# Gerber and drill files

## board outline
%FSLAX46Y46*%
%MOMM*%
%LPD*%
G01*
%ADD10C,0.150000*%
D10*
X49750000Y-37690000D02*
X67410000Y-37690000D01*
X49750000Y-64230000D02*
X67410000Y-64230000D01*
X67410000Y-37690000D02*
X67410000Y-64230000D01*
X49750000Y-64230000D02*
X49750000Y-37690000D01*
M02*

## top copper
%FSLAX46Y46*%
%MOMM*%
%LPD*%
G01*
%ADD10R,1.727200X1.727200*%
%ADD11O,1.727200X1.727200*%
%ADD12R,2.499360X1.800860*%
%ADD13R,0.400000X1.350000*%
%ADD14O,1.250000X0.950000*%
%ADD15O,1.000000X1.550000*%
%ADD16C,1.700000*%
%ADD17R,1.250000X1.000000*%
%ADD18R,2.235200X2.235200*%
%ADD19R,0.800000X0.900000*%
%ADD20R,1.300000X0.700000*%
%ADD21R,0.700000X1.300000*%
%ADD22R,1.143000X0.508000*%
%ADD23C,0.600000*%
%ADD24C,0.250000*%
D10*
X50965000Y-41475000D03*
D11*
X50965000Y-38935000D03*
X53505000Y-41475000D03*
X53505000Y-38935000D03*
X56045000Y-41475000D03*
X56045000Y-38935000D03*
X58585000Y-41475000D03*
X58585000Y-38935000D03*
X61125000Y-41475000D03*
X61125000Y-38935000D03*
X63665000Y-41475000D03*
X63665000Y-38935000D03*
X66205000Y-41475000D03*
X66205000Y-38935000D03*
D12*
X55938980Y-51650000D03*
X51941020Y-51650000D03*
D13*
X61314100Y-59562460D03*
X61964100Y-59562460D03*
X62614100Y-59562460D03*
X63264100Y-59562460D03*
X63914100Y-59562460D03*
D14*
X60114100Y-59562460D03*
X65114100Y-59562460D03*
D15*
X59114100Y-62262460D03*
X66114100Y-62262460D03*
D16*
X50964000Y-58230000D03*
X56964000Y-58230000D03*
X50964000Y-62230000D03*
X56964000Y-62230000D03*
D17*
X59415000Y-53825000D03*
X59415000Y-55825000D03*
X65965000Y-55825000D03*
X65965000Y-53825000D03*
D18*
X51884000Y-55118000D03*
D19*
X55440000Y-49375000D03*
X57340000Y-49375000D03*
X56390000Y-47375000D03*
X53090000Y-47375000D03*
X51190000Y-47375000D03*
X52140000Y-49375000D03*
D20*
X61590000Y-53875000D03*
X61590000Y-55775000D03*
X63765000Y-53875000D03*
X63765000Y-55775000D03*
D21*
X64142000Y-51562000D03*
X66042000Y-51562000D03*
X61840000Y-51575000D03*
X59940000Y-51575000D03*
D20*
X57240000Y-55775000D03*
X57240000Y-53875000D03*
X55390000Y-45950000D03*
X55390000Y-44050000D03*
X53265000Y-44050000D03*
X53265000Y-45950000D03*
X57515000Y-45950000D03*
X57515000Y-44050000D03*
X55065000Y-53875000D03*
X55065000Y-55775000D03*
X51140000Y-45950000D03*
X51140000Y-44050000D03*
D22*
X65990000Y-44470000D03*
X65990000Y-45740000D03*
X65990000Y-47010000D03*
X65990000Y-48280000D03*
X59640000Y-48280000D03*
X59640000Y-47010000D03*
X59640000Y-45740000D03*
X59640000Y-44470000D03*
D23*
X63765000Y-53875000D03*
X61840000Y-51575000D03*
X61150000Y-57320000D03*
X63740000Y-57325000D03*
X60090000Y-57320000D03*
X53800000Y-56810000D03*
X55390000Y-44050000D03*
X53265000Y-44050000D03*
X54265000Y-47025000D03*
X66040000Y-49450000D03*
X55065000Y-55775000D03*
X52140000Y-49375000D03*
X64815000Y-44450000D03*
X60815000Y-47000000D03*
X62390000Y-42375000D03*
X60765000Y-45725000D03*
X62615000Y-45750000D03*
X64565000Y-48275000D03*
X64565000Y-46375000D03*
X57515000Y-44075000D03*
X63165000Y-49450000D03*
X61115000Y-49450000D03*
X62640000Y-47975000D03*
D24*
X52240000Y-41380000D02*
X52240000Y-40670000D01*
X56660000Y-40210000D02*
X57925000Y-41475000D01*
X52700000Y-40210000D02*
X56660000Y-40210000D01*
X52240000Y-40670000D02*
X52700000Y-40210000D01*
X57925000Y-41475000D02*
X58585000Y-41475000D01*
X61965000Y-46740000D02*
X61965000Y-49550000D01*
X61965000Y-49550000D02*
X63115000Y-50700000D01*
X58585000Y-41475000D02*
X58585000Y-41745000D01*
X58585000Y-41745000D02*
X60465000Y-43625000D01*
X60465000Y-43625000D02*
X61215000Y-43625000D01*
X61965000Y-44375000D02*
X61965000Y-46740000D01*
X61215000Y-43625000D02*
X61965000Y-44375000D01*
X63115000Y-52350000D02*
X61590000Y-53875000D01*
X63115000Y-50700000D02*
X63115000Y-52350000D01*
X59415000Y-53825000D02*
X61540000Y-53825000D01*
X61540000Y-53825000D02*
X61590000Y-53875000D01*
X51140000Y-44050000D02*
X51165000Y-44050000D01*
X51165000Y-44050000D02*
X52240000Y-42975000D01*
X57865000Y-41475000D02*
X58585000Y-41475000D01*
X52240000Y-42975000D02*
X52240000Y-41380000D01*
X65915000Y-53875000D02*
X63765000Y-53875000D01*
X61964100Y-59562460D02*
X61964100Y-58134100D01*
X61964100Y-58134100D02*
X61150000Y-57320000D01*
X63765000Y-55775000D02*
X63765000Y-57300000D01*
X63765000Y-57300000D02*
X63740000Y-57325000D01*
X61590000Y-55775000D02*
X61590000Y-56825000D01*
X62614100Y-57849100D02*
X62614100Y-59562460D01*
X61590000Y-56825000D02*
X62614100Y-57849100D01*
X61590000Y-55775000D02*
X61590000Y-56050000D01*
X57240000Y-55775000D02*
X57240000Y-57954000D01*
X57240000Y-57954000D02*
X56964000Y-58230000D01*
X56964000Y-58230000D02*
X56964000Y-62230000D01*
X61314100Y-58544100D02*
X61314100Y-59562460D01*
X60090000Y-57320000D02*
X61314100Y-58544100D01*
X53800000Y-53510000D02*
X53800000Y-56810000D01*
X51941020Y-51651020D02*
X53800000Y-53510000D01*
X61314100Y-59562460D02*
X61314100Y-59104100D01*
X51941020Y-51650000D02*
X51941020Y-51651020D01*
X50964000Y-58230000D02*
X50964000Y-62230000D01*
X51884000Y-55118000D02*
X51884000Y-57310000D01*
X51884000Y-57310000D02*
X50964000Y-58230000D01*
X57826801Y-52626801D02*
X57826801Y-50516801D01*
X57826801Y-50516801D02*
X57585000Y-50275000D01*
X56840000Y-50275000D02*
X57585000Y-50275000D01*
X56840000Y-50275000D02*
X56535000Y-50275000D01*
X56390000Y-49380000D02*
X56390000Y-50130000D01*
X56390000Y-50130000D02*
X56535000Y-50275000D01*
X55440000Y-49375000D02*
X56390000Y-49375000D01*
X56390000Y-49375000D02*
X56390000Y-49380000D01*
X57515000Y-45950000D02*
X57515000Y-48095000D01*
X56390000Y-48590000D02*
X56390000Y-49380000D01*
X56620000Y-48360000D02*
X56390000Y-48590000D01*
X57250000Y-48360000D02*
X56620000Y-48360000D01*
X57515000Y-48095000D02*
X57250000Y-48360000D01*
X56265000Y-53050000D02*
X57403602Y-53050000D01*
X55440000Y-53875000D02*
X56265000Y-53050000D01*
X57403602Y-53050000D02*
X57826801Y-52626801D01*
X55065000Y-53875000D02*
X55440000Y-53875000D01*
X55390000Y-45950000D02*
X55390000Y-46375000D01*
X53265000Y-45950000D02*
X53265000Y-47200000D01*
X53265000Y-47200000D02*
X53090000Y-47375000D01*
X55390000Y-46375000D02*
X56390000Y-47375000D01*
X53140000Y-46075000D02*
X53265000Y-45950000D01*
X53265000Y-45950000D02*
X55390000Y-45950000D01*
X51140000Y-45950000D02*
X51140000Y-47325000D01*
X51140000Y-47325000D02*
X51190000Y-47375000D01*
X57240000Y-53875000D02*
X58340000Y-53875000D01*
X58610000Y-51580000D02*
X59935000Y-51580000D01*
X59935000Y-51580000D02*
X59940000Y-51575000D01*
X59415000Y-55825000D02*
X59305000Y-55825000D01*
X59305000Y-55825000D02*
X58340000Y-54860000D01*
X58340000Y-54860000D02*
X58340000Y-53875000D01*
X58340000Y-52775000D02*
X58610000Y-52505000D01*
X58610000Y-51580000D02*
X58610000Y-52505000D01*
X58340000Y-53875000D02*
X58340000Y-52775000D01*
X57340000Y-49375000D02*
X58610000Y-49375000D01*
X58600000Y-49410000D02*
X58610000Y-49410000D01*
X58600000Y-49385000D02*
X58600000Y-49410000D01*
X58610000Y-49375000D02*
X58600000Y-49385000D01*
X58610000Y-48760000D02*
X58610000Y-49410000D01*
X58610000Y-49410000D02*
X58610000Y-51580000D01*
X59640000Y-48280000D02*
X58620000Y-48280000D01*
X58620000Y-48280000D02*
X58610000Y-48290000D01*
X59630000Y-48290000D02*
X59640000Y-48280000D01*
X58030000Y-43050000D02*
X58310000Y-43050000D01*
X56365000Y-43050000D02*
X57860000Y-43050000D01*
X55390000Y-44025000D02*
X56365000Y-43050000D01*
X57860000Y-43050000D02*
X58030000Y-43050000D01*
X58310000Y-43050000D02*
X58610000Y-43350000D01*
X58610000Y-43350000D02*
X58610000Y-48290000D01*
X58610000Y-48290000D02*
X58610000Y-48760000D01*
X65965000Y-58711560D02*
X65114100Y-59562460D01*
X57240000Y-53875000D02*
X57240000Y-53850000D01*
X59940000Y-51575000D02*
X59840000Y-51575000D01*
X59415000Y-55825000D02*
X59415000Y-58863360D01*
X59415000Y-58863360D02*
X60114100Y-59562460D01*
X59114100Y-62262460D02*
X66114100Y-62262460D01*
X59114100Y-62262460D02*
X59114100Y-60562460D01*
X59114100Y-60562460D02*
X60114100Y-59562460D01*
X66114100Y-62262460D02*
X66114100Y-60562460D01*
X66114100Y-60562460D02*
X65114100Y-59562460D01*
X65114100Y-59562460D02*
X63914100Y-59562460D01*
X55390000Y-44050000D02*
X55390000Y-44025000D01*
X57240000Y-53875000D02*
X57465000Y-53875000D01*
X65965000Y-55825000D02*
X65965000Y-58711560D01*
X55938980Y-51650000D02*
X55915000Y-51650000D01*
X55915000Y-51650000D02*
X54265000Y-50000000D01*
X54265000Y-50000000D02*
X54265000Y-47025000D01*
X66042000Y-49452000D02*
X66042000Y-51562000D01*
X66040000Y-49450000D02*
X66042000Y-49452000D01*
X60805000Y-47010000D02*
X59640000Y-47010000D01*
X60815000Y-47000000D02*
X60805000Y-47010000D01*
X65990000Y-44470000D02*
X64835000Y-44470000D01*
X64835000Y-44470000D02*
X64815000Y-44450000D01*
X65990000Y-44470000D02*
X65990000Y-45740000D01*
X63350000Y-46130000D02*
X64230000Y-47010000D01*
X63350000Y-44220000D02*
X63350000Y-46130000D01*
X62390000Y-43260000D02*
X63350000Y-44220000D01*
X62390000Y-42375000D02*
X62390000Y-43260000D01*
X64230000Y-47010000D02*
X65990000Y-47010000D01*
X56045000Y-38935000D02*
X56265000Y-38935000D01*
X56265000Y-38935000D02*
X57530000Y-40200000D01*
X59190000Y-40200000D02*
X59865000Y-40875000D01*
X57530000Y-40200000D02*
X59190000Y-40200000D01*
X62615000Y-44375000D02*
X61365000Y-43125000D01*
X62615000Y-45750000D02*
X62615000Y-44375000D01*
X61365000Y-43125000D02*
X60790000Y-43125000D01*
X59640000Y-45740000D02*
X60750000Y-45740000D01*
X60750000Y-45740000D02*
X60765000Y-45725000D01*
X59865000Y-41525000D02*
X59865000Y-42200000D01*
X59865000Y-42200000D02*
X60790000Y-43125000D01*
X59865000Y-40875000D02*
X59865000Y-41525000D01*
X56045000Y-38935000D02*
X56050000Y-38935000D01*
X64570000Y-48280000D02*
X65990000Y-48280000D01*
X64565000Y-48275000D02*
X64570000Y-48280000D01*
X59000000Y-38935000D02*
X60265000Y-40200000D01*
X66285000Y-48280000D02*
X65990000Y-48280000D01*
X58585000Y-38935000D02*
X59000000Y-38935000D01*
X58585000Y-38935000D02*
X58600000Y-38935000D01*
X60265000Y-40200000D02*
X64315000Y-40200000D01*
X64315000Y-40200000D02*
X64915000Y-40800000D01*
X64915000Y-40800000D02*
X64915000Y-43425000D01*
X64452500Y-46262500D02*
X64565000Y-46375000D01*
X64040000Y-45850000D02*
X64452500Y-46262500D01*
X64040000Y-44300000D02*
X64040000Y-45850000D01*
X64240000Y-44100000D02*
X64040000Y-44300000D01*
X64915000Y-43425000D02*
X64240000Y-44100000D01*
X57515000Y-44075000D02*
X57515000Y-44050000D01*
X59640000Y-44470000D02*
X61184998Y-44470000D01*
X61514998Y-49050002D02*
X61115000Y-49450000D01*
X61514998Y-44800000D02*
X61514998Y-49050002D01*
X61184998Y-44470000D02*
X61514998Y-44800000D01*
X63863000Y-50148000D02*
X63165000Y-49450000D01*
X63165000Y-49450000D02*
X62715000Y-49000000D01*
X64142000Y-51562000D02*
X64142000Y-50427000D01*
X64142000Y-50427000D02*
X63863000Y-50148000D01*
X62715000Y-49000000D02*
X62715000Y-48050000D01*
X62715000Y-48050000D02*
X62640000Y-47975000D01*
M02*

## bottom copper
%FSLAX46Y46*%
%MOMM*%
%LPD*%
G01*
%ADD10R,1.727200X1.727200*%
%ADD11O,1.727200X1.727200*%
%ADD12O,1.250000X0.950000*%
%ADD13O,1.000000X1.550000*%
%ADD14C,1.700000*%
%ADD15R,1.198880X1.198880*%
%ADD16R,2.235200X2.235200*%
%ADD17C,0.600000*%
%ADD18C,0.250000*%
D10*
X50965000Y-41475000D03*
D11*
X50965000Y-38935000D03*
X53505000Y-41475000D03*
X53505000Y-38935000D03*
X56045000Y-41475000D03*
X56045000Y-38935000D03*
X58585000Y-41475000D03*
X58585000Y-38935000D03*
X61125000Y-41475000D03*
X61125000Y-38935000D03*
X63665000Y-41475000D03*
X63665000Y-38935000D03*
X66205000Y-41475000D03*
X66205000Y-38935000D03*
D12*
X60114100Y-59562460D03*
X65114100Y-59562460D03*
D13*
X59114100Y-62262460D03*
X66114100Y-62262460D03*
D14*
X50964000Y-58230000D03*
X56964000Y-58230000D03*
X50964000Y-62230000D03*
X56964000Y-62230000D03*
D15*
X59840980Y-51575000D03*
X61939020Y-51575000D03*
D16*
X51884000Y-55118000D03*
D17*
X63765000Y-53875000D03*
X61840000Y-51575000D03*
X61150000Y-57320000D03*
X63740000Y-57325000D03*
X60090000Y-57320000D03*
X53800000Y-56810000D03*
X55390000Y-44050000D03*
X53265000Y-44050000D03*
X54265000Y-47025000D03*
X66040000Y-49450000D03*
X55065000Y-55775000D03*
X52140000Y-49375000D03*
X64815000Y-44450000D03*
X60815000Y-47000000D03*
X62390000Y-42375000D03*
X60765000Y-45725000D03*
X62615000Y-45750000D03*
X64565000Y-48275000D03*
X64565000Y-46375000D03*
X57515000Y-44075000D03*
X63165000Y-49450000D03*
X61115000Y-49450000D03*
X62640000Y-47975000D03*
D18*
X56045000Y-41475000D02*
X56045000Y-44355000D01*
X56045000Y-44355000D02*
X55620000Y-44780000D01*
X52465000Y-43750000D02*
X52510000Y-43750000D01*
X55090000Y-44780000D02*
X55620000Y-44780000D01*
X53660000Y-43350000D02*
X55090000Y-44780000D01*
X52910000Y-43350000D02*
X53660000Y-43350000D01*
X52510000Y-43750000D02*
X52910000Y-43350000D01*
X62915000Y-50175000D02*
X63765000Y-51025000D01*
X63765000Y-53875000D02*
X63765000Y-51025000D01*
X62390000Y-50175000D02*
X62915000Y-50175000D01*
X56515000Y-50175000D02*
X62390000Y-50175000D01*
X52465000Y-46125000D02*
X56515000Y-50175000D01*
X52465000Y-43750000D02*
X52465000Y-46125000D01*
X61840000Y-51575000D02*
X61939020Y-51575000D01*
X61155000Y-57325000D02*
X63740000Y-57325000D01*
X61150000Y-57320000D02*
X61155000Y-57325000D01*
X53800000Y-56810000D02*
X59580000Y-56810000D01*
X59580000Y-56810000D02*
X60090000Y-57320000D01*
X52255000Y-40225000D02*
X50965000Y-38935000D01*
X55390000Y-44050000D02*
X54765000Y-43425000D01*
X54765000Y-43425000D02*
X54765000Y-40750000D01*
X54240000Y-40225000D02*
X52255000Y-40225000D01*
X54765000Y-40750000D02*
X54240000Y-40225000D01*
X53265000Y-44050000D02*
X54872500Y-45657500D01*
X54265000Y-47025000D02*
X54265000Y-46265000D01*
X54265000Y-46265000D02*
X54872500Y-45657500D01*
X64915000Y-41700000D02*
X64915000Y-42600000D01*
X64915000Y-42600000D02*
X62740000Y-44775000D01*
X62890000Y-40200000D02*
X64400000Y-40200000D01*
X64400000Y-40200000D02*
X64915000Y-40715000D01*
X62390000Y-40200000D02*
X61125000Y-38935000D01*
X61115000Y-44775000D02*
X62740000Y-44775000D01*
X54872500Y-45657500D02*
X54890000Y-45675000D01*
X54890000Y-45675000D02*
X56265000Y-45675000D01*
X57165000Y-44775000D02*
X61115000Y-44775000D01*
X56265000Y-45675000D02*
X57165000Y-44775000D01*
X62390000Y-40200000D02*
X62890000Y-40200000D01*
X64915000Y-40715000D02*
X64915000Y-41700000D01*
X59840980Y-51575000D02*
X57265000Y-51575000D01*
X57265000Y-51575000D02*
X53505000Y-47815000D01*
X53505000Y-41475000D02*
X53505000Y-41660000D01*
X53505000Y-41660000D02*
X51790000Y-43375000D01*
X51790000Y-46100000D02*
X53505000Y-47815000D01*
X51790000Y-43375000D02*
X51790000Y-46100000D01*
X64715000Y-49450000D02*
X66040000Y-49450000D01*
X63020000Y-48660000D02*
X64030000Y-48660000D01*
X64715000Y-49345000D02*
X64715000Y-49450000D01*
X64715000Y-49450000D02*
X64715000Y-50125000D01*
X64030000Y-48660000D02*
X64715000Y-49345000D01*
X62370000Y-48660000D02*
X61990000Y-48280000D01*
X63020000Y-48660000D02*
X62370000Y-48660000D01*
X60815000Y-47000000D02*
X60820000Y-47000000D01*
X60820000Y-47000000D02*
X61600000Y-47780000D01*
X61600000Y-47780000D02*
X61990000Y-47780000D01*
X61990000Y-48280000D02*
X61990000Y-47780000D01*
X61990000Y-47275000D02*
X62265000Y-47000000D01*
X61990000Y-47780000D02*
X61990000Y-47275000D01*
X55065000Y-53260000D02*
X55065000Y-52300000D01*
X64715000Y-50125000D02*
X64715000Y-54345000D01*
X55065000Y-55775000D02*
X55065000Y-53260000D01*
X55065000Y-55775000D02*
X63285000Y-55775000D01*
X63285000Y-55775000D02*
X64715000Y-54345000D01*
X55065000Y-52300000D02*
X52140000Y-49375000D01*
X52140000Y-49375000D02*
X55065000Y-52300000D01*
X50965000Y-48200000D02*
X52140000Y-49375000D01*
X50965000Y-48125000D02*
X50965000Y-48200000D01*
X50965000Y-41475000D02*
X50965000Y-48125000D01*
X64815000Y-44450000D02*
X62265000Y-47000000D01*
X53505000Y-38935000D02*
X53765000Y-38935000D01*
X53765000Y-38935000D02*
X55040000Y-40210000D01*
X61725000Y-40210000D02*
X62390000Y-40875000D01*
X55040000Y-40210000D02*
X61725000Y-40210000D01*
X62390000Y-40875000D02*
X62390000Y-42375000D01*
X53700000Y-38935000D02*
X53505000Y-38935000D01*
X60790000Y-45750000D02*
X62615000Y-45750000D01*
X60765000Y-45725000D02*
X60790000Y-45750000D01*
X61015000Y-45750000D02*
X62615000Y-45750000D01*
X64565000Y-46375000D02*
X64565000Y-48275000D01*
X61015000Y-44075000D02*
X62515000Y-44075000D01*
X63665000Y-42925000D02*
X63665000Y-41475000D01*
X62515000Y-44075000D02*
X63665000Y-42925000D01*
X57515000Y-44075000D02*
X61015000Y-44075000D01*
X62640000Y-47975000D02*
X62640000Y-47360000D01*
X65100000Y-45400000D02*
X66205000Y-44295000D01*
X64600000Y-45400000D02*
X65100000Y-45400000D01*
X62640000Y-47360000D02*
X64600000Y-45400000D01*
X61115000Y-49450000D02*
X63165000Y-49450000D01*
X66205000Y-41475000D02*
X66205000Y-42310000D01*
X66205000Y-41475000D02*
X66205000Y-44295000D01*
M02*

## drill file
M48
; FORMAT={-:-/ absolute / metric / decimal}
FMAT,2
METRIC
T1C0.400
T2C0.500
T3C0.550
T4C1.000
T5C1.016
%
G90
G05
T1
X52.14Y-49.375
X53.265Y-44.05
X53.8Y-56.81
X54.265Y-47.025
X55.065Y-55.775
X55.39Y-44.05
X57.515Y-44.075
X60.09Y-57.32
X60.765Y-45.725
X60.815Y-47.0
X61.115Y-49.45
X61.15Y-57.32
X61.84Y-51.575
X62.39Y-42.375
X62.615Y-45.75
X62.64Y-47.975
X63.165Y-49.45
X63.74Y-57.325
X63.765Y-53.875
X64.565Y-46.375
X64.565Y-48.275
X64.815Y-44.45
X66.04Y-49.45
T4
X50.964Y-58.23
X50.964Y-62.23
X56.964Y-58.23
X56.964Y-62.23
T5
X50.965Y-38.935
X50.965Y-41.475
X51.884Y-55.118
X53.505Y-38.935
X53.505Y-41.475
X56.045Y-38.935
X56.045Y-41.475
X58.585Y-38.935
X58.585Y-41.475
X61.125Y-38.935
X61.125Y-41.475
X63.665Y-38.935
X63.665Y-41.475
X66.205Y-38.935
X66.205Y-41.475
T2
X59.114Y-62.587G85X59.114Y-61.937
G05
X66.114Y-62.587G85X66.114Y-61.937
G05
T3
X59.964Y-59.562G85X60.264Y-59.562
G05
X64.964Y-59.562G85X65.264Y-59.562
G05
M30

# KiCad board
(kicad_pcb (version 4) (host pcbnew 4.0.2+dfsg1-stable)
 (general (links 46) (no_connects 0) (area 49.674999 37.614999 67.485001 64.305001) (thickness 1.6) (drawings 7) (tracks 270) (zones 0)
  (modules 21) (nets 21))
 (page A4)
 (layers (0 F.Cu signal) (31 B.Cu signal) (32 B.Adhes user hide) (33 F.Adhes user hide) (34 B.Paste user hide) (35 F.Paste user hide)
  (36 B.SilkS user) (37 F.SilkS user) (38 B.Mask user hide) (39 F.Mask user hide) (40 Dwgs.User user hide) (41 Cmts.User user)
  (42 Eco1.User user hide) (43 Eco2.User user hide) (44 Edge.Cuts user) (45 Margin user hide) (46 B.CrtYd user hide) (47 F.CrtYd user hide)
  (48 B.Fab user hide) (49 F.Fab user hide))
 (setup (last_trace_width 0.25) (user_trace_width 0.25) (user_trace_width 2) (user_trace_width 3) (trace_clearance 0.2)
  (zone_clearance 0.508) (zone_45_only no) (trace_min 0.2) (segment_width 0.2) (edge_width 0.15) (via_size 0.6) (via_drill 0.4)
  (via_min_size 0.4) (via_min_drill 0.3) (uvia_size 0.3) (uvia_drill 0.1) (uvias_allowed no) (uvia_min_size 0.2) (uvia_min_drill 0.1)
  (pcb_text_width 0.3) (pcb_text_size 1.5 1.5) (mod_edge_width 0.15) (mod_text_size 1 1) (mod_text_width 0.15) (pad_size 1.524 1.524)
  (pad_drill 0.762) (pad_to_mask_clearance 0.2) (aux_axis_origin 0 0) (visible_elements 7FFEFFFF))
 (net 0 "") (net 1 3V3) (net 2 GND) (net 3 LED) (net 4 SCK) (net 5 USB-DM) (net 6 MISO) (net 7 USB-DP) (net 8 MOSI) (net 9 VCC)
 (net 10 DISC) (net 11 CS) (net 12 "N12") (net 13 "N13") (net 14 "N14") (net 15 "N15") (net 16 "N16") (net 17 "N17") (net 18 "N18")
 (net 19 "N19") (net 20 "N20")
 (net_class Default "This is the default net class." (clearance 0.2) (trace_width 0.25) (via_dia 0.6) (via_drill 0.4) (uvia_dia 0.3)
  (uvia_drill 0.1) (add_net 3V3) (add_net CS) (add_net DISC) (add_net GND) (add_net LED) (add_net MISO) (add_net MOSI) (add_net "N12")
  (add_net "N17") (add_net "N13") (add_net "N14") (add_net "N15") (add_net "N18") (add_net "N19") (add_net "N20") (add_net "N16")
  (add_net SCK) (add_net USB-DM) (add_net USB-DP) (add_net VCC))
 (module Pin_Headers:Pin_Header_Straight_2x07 (layer F.Cu) (at 50.965 41.475 90)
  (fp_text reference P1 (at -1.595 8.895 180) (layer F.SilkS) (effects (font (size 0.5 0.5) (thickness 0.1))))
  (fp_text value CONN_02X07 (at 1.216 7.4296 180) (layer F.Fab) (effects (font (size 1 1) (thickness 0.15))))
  (pad 1 thru_hole rect (at 0 0 90) (size 1.7272 1.7272) (drill 1.016) (layers *.Cu *.Mask) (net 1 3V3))
  (pad 2 thru_hole oval (at 2.54 0 90) (size 1.7272 1.7272) (drill 1.016) (layers *.Cu *.Mask) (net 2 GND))
  (pad 3 thru_hole oval (at 0 2.54 90) (size 1.7272 1.7272) (drill 1.016) (layers *.Cu *.Mask) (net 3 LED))
  (pad 4 thru_hole oval (at 2.54 2.54 90) (size 1.7272 1.7272) (drill 1.016) (layers *.Cu *.Mask) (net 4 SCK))
  (pad 5 thru_hole oval (at 0 5.08 90) (size 1.7272 1.7272) (drill 1.016) (layers *.Cu *.Mask) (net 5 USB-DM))
  (pad 6 thru_hole oval (at 2.54 5.08 90) (size 1.7272 1.7272) (drill 1.016) (layers *.Cu *.Mask) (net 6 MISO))
  (pad 7 thru_hole oval (at 0 7.62 90) (size 1.7272 1.7272) (drill 1.016) (layers *.Cu *.Mask) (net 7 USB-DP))
  (pad 8 thru_hole oval (at 2.54 7.62 90) (size 1.7272 1.7272) (drill 1.016) (layers *.Cu *.Mask) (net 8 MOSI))
  (pad 9 thru_hole oval (at 0 10.16 90) (size 1.7272 1.7272) (drill 1.016) (layers *.Cu *.Mask))
  (pad 10 thru_hole oval (at 2.54 10.16 90) (size 1.7272 1.7272) (drill 1.016) (layers *.Cu *.Mask) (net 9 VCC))
  (pad 11 thru_hole oval (at 0 12.7 90) (size 1.7272 1.7272) (drill 1.016) (layers *.Cu *.Mask) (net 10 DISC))
  (pad 12 thru_hole oval (at 2.54 12.7 90) (size 1.7272 1.7272) (drill 1.016) (layers *.Cu *.Mask))
  (pad 13 thru_hole oval (at 0 15.24 90) (size 1.7272 1.7272) (drill 1.016) (layers *.Cu *.Mask) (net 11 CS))
  (pad 14 thru_hole oval (at 2.54 15.24 90) (size 1.7272 1.7272) (drill 1.016) (layers *.Cu *.Mask)))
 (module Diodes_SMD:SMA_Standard (layer F.Cu) (at 53.94 51.65 180)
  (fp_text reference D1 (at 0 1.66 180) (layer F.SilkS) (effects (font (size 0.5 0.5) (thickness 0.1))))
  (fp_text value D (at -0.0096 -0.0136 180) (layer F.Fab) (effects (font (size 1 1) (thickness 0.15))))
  (pad 1 smd rect (at -1.99898 0 180) (size 2.49936 1.80086) (layers F.Cu F.Paste F.Mask) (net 9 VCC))
  (pad 2 smd rect (at 1.99898 0 180) (size 2.49936 1.80086) (layers F.Cu F.Paste F.Mask) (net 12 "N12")))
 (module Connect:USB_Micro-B (layer F.Cu) (at 62.615 61.125)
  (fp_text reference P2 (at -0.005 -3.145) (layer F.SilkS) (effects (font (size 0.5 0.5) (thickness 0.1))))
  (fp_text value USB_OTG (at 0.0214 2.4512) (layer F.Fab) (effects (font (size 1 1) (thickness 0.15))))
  (pad 1 smd rect (at -1.3009 -1.56254 90) (size 1.35 0.4) (layers F.Cu F.Paste F.Mask) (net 12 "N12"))
  (pad 2 smd rect (at -0.6509 -1.56254 90) (size 1.35 0.4) (layers F.Cu F.Paste F.Mask) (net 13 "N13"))
  (pad 3 smd rect (at -0.0009 -1.56254 90) (size 1.35 0.4) (layers F.Cu F.Paste F.Mask) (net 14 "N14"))
  (pad 4 smd rect (at 0.6491 -1.56254 90) (size 1.35 0.4) (layers F.Cu F.Paste F.Mask))
  (pad 5 smd rect (at 1.2991 -1.56254 90) (size 1.35 0.4) (layers F.Cu F.Paste F.Mask) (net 2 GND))
  (pad 6 thru_hole oval (at -2.5009 -1.56254 90) (size 0.95 1.25) (drill oval 0.55 0.85) (layers *.Cu *.Mask) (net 2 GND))
  (pad 6 thru_hole oval (at 2.4991 -1.56254 90) (size 0.95 1.25) (drill oval 0.55 0.85) (layers *.Cu *.Mask) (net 2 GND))
  (pad 6 thru_hole oval (at -3.5009 1.13746 90) (size 1.55 1) (drill oval 1.15 0.5) (layers *.Cu *.Mask) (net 2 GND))
  (pad 6 thru_hole oval (at 3.4991 1.13746 90) (size 1.55 1) (drill oval 1.15 0.5) (layers *.Cu *.Mask) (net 2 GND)))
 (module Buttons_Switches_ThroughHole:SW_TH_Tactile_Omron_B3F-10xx (layer F.Cu) (at 56.964 62.23 180)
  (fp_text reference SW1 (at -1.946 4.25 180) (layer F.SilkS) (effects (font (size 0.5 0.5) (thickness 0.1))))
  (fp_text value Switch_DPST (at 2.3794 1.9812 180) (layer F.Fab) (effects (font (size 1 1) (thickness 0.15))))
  (pad 4 thru_hole circle (at 6 4 180) (size 1.7 1.7) (drill 1) (layers *.Cu *.Mask) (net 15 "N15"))
  (pad 3 thru_hole circle (at 0 4 180) (size 1.7 1.7) (drill 1) (layers *.Cu *.Mask) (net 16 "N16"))
  (pad 2 thru_hole circle (at 6 0 180) (size 1.7 1.7) (drill 1) (layers *.Cu *.Mask) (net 15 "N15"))
  (pad 1 thru_hole circle (at 0 0 180) (size 1.7 1.7) (drill 1) (layers *.Cu *.Mask) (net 16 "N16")))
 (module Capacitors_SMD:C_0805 (layer F.Cu) (at 59.415 54.825 270)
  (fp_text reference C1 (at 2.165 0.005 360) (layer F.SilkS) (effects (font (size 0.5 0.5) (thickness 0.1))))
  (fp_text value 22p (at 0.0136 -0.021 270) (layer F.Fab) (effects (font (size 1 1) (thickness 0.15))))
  (pad 1 smd rect (at -1 0 270) (size 1 1.25) (layers F.Cu F.Paste F.Mask) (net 7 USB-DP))
  (pad 2 smd rect (at 1 0 270) (size 1 1.25) (layers F.Cu F.Paste F.Mask) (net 2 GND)))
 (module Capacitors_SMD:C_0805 (layer F.Cu) (at 65.965 54.825 90)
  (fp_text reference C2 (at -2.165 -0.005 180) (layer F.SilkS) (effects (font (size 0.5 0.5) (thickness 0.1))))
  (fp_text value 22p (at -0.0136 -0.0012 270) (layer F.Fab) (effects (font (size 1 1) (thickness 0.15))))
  (pad 1 smd rect (at -1 0 90) (size 1 1.25) (layers F.Cu F.Paste F.Mask) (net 2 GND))
  (pad 2 smd rect (at 1 0 90) (size 1 1.25) (layers F.Cu F.Paste F.Mask) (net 5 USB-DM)))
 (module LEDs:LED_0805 (layer B.Cu) (at 60.89 51.575 180)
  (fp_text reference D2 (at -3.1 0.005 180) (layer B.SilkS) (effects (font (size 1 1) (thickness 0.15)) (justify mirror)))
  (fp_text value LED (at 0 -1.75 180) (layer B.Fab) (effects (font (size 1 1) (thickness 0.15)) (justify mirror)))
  (pad 2 smd rect (at 1.04902 0) (size 1.19888 1.19888) (layers B.Cu B.Paste B.Mask) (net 3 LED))
  (pad 1 smd rect (at -1.04902 0) (size 1.19888 1.19888) (layers B.Cu B.Paste B.Mask) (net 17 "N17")))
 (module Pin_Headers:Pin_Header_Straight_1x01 (layer F.Cu) (at 51.884 55.118)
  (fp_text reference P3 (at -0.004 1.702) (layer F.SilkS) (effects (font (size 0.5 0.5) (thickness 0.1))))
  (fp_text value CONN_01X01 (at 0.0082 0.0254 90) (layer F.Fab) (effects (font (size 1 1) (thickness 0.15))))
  (pad 1 thru_hole rect (at 0 0) (size 2.2352 2.2352) (drill 1.016) (layers *.Cu *.Mask) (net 15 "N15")))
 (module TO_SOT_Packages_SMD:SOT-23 (layer F.Cu) (at 56.39 48.375 90)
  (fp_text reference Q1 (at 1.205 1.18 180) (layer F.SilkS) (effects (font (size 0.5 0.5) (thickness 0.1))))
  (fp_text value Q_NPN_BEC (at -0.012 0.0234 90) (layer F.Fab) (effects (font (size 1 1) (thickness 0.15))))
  (pad 1 smd rect (at -1 -0.95 90) (size 0.9 0.8) (layers F.Cu F.Paste F.Mask) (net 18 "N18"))
  (pad 2 smd rect (at -1 0.95 90) (size 0.9 0.8) (layers F.Cu F.Paste F.Mask) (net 2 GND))
  (pad 3 smd rect (at 1 0 90) (size 0.9 0.8) (layers F.Cu F.Paste F.Mask) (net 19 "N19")))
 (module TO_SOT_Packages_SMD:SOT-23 (layer F.Cu) (at 52.14 48.375 270)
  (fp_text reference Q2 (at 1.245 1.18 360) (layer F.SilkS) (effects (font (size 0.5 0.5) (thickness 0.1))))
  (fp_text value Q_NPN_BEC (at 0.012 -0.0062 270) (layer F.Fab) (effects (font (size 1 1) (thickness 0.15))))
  (pad 1 smd rect (at -1 -0.95 270) (size 0.9 0.8) (layers F.Cu F.Paste F.Mask) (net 19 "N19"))
  (pad 2 smd rect (at -1 0.95 270) (size 0.9 0.8) (layers F.Cu F.Paste F.Mask) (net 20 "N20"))
  (pad 3 smd rect (at 1 0 270) (size 0.9 0.8) (layers F.Cu F.Paste F.Mask) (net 1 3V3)))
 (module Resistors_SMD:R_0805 (layer F.Cu) (at 61.59 54.825 270)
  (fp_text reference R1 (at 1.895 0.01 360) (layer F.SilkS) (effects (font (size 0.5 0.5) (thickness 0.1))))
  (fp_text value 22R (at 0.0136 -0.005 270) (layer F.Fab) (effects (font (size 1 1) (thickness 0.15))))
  (pad 1 smd rect (at -0.95 0 270) (size 0.7 1.3) (layers F.Cu F.Paste F.Mask) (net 7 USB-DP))
  (pad 2 smd rect (at 0.95 0 270) (size 0.7 1.3) (layers F.Cu F.Paste F.Mask) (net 14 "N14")))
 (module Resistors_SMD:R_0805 (layer F.Cu) (at 63.765 54.825 270)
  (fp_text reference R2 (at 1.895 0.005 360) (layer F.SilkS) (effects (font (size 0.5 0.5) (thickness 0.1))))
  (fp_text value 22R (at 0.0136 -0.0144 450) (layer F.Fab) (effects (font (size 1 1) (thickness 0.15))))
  (pad 1 smd rect (at -0.95 0 270) (size 0.7 1.3) (layers F.Cu F.Paste F.Mask) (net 5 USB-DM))
  (pad 2 smd rect (at 0.95 0 270) (size 0.7 1.3) (layers F.Cu F.Paste F.Mask) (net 13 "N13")))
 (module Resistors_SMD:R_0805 (layer F.Cu) (at 65.092 51.562)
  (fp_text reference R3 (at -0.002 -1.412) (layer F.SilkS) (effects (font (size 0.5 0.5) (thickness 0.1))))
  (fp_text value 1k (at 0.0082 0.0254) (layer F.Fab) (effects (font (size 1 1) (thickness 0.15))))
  (pad 1 smd rect (at -0.95 0) (size 0.7 1.3) (layers F.Cu F.Paste F.Mask) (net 11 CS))
  (pad 2 smd rect (at 0.95 0) (size 0.7 1.3) (layers F.Cu F.Paste F.Mask) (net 1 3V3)))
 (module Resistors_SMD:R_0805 (layer F.Cu) (at 60.89 51.575 180)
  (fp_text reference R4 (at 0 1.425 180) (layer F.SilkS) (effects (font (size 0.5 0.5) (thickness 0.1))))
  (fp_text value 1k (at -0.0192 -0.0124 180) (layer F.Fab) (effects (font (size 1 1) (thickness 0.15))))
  (pad 1 smd rect (at -0.95 0 180) (size 0.7 1.3) (layers F.Cu F.Paste F.Mask) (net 17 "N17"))
  (pad 2 smd rect (at 0.95 0 180) (size 0.7 1.3) (layers F.Cu F.Paste F.Mask) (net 2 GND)))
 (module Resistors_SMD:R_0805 (layer F.Cu) (at 57.24 54.825 90)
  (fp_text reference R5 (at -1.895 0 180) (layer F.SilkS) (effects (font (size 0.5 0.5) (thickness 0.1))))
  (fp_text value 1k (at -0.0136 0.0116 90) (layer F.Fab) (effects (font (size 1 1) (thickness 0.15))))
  (pad 1 smd rect (at -0.95 0 90) (size 0.7 1.3) (layers F.Cu F.Paste F.Mask) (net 16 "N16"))
  (pad 2 smd rect (at 0.95 0 90) (size 0.7 1.3) (layers F.Cu F.Paste F.Mask) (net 2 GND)))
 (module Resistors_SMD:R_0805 (layer F.Cu) (at 55.39 45 90)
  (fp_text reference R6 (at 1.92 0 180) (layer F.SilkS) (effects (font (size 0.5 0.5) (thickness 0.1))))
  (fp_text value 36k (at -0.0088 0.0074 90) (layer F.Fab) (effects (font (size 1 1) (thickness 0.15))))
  (pad 1 smd rect (at -0.95 0 90) (size 0.7 1.3) (layers F.Cu F.Paste F.Mask) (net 19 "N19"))
  (pad 2 smd rect (at 0.95 0 90) (size 0.7 1.3) (layers F.Cu F.Paste F.Mask) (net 2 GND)))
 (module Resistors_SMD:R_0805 (layer F.Cu) (at 53.265 45 270)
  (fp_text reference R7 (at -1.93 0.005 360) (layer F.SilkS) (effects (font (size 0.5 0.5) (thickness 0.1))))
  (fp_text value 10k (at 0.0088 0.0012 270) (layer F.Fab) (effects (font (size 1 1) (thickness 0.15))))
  (pad 1 smd rect (at -0.95 0 270) (size 0.7 1.3) (layers F.Cu F.Paste F.Mask) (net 9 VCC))
  (pad 2 smd rect (at 0.95 0 270) (size 0.7 1.3) (layers F.Cu F.Paste F.Mask) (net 19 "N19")))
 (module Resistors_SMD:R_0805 (layer F.Cu) (at 57.515 45 90)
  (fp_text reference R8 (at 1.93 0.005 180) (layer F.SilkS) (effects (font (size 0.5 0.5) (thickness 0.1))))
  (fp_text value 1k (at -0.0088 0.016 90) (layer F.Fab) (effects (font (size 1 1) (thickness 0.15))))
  (pad 1 smd rect (at -0.95 0 90) (size 0.7 1.3) (layers F.Cu F.Paste F.Mask) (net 18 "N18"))
  (pad 2 smd rect (at 0.95 0 90) (size 0.7 1.3) (layers F.Cu F.Paste F.Mask) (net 10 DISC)))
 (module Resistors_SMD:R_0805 (layer F.Cu) (at 55.065 54.825 270)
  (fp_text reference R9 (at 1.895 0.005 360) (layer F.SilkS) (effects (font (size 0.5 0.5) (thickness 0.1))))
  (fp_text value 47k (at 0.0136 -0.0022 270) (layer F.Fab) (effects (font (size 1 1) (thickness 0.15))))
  (pad 1 smd rect (at -0.95 0 270) (size 0.7 1.3) (layers F.Cu F.Paste F.Mask) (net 18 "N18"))
  (pad 2 smd rect (at 0.95 0 270) (size 0.7 1.3) (layers F.Cu F.Paste F.Mask) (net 1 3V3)))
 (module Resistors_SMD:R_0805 (layer F.Cu) (at 51.14 45 90)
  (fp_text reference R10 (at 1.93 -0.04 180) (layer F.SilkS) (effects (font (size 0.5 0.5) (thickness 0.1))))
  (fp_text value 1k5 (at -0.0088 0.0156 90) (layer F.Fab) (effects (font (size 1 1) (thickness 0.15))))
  (pad 1 smd rect (at -0.95 0 90) (size 0.7 1.3) (layers F.Cu F.Paste F.Mask) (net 20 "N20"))
  (pad 2 smd rect (at 0.95 0 90) (size 0.7 1.3) (layers F.Cu F.Paste F.Mask) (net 7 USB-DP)))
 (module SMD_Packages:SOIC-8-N (layer F.Cu) (at 62.815 46.375 270)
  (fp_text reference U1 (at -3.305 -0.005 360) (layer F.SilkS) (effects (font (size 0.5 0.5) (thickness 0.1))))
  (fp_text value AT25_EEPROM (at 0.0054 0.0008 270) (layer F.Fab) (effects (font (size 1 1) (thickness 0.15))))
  (pad 8 smd rect (at -1.905 -3.175 270) (size 0.508 1.143) (layers F.Cu F.Paste F.Mask) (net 1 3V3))
  (pad 7 smd rect (at -0.635 -3.175 270) (size 0.508 1.143) (layers F.Cu F.Paste F.Mask) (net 1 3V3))
  (pad 6 smd rect (at 0.635 -3.175 270) (size 0.508 1.143) (layers F.Cu F.Paste F.Mask) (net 4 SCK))
  (pad 5 smd rect (at 1.905 -3.175 270) (size 0.508 1.143) (layers F.Cu F.Paste F.Mask) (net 8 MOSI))
  (pad 4 smd rect (at 1.905 3.175 270) (size 0.508 1.143) (layers F.Cu F.Paste F.Mask) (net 2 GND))
  (pad 3 smd rect (at 0.635 3.175 270) (size 0.508 1.143) (layers F.Cu F.Paste F.Mask) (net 1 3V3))
  (pad 2 smd rect (at -0.635 3.175 270) (size 0.508 1.143) (layers F.Cu F.Paste F.Mask) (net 6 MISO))
  (pad 1 smd rect (at -1.905 3.175 270) (size 0.508 1.143) (layers F.Cu F.Paste F.Mask) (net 11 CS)))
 (gr_line (start 49.75 37.69) (end 67.41 37.69) (angle 90) (layer Edge.Cuts) (width 0.15))
 (gr_line (start 49.75 64.23) (end 67.41 64.23) (angle 90) (layer Edge.Cuts) (width 0.15))
 (gr_line (start 67.41 37.69) (end 67.41 64.23) (angle 90) (layer Edge.Cuts) (width 0.15))
 (gr_line (start 49.75 64.23) (end 49.75 37.69) (angle 90) (layer Edge.Cuts) (width 0.15))
 (segment (start 52.24 41.38) (end 52.24 40.67) (width 0.25) (layer F.Cu) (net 7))
 (segment (start 56.66 40.21) (end 57.925 41.475) (width 0.25) (layer F.Cu) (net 7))
 (segment (start 52.7 40.21) (end 56.66 40.21) (width 0.25) (layer F.Cu) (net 7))
 (segment (start 52.24 40.67) (end 52.7 40.21) (width 0.25) (layer F.Cu) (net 7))
 (segment (start 57.925 41.475) (end 58.585 41.475) (width 0.25) (layer F.Cu) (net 7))
 (segment (start 61.965 46.74) (end 61.965 49.55) (width 0.25) (layer F.Cu) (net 7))
 (segment (start 61.965 49.55) (end 63.115 50.7) (width 0.25) (layer F.Cu) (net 7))
 (segment (start 58.585 41.475) (end 58.585 41.745) (width 0.25) (layer F.Cu) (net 7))
 (segment (start 58.585 41.745) (end 60.465 43.625) (width 0.25) (layer F.Cu) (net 7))
 (segment (start 60.465 43.625) (end 61.215 43.625) (width 0.25) (layer F.Cu) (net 7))
 (segment (start 61.965 44.375) (end 61.965 46.74) (width 0.25) (layer F.Cu) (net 7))
 (segment (start 61.215 43.625) (end 61.965 44.375) (width 0.25) (layer F.Cu) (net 7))
 (segment (start 63.115 52.35) (end 61.59 53.875) (width 0.25) (layer F.Cu) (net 7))
 (segment (start 63.115 50.7) (end 63.115 52.35) (width 0.25) (layer F.Cu) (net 7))
 (segment (start 59.415 53.825) (end 61.54 53.825) (width 0.25) (layer F.Cu) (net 7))
 (segment (start 61.54 53.825) (end 61.59 53.875) (width 0.25) (layer F.Cu) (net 7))
 (segment (start 51.14 44.05) (end 51.165 44.05) (width 0.25) (layer F.Cu) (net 7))
 (segment (start 51.165 44.05) (end 52.24 42.975) (width 0.25) (layer F.Cu) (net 7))
 (segment (start 57.865 41.475) (end 58.585 41.475) (width 0.25) (layer F.Cu) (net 7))
 (segment (start 52.24 42.975) (end 52.24 41.38) (width 0.25) (layer F.Cu) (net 7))
 (segment (start 56.045 41.475) (end 56.045 44.355) (width 0.25) (layer B.Cu) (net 5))
 (segment (start 56.045 44.355) (end 55.62 44.78) (width 0.25) (layer B.Cu) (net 5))
 (segment (start 52.465 43.75) (end 52.51 43.75) (width 0.25) (layer B.Cu) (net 5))
 (segment (start 55.09 44.78) (end 55.62 44.78) (width 0.25) (layer B.Cu) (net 5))
 (segment (start 53.66 43.35) (end 55.09 44.78) (width 0.25) (layer B.Cu) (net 5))
 (segment (start 52.91 43.35) (end 53.66 43.35) (width 0.25) (layer B.Cu) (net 5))
 (segment (start 52.51 43.75) (end 52.91 43.35) (width 0.25) (layer B.Cu) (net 5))
 (segment (start 62.915 50.175) (end 63.765 51.025) (width 0.25) (layer B.Cu) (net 5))
 (segment (start 63.765 53.875) (end 63.765 51.025) (width 0.25) (layer B.Cu) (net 5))
 (via (at 63.765 53.875) (size 0.6) (drill 0.4) (layers F.Cu B.Cu) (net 5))
 (segment (start 65.915 53.875) (end 63.765 53.875) (width 0.25) (layer F.Cu) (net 5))
 (segment (start 62.39 50.175) (end 62.915 50.175) (width 0.25) (layer B.Cu) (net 5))
 (segment (start 56.515 50.175) (end 62.39 50.175) (width 0.25) (layer B.Cu) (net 5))
 (segment (start 52.465 46.125) (end 56.515 50.175) (width 0.25) (layer B.Cu) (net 5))
 (segment (start 52.465 43.75) (end 52.465 46.125) (width 0.25) (layer B.Cu) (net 5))
 (via (at 61.84 51.575) (size 0.6) (drill 0.4) (layers F.Cu B.Cu) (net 17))
 (segment (start 61.84 51.575) (end 61.93902 51.575) (width 0.25) (layer B.Cu) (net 17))
 (segment (start 61.9641 59.56246) (end 61.9641 58.1341) (width 0.25) (layer F.Cu) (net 13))
 (segment (start 61.155 57.325) (end 63.74 57.325) (width 0.25) (layer B.Cu) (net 13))
 (segment (start 61.15 57.32) (end 61.155 57.325) (width 0.25) (layer B.Cu) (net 13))
 (via (at 61.15 57.32) (size 0.6) (drill 0.4) (layers F.Cu B.Cu) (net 13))
 (segment (start 61.9641 58.1341) (end 61.15 57.32) (width 0.25) (layer F.Cu) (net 13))
 (segment (start 63.765 55.775) (end 63.765 57.3) (width 0.25) (layer F.Cu) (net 13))
 (via (at 63.74 57.325) (size 0.6) (drill 0.4) (layers F.Cu B.Cu) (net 13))
 (segment (start 63.765 57.3) (end 63.74 57.325) (width 0.25) (layer F.Cu) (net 13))
 (segment (start 61.59 55.775) (end 61.59 56.825) (width 0.25) (layer F.Cu) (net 14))
 (segment (start 62.6141 57.8491) (end 62.6141 59.56246) (width 0.25) (layer F.Cu) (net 14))
 (segment (start 61.59 56.825) (end 62.6141 57.8491) (width 0.25) (layer F.Cu) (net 14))
 (segment (start 61.59 55.775) (end 61.59 56.05) (width 0.25) (layer F.Cu) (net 14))
 (segment (start 57.24 55.775) (end 57.24 57.954) (width 0.25) (layer F.Cu) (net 16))
 (segment (start 57.24 57.954) (end 56.964 58.23) (width 0.25) (layer F.Cu) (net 16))
 (segment (start 56.964 58.23) (end 56.964 62.23) (width 0.25) (layer F.Cu) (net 16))
 (segment (start 53.8 56.81) (end 59.58 56.81) (width 0.25) (layer B.Cu) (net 12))
 (segment (start 61.3141 58.5441) (end 61.3141 59.56246) (width 0.25) (layer F.Cu) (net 12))
 (segment (start 60.09 57.32) (end 61.3141 58.5441) (width 0.25) (layer F.Cu) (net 12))
 (via (at 60.09 57.32) (size 0.6) (drill 0.4) (layers F.Cu B.Cu) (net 12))
 (segment (start 59.58 56.81) (end 60.09 57.32) (width 0.25) (layer B.Cu) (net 12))
 (via (at 53.8 56.81) (size 0.6) (drill 0.4) (layers F.Cu B.Cu) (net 12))
 (segment (start 53.8 53.51) (end 53.8 56.81) (width 0.25) (layer F.Cu) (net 12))
 (segment (start 51.94102 51.65102) (end 53.8 53.51) (width 0.25) (layer F.Cu) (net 12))
 (segment (start 61.3141 59.56246) (end 61.3141 59.1041) (width 0.25) (layer F.Cu) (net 12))
 (segment (start 51.94102 51.65) (end 51.94102 51.65102) (width 0.25) (layer F.Cu) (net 12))
 (segment (start 50.964 58.23) (end 50.964 62.23) (width 0.25) (layer F.Cu) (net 15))
 (segment (start 51.884 55.118) (end 51.884 57.31) (width 0.25) (layer F.Cu) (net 15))
 (segment (start 51.884 57.31) (end 50.964 58.23) (width 0.25) (layer F.Cu) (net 15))
 (segment (start 57.826801 52.626801) (end 57.826801 50.516801) (width 0.25) (layer F.Cu) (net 18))
 (segment (start 57.826801 50.516801) (end 57.585 50.275) (width 0.25) (layer F.Cu) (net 18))
 (segment (start 56.84 50.275) (end 57.585 50.275) (width 0.25) (layer F.Cu) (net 18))
 (segment (start 56.84 50.275) (end 56.535 50.275) (width 0.25) (layer F.Cu) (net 18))
 (segment (start 56.39 49.38) (end 56.39 50.13) (width 0.25) (layer F.Cu) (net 18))
 (segment (start 56.39 50.13) (end 56.535 50.275) (width 0.25) (layer F.Cu) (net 18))
 (segment (start 55.44 49.375) (end 56.39 49.375) (width 0.25) (layer F.Cu) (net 18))
 (segment (start 56.39 49.375) (end 56.39 49.38) (width 0.25) (layer F.Cu) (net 18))
 (segment (start 57.515 45.95) (end 57.515 48.095) (width 0.25) (layer F.Cu) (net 18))
 (segment (start 56.39 48.59) (end 56.39 49.38) (width 0.25) (layer F.Cu) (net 18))
 (segment (start 56.62 48.36) (end 56.39 48.59) (width 0.25) (layer F.Cu) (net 18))
 (segment (start 57.25 48.36) (end 56.62 48.36) (width 0.25) (layer F.Cu) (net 18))
 (segment (start 57.515 48.095) (end 57.25 48.36) (width 0.25) (layer F.Cu) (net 18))
 (segment (start 56.265 53.05) (end 57.403602 53.05) (width 0.25) (layer F.Cu) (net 18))
 (segment (start 55.44 53.875) (end 56.265 53.05) (width 0.25) (layer F.Cu) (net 18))
 (segment (start 57.403602 53.05) (end 57.826801 52.626801) (width 0.25) (layer F.Cu) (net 18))
 (segment (start 55.065 53.875) (end 55.44 53.875) (width 0.25) (layer F.Cu) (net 18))
 (segment (start 55.39 45.95) (end 55.39 46.375) (width 0.25) (layer F.Cu) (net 19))
 (segment (start 53.265 45.95) (end 53.265 47.2) (width 0.25) (layer F.Cu) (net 19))
 (segment (start 53.265 47.2) (end 53.09 47.375) (width 0.25) (layer F.Cu) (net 19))
 (segment (start 55.39 46.375) (end 56.39 47.375) (width 0.25) (layer F.Cu) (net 19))
 (segment (start 53.14 46.075) (end 53.265 45.95) (width 0.25) (layer F.Cu) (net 19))
 (segment (start 53.265 45.95) (end 55.39 45.95) (width 0.25) (layer F.Cu) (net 19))
 (segment (start 51.14 45.95) (end 51.14 47.325) (width 0.25) (layer F.Cu) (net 20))
 (segment (start 51.14 47.325) (end 51.19 47.375) (width 0.25) (layer F.Cu) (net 20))
 (segment (start 57.24 53.875) (end 58.34 53.875) (width 0.25) (layer F.Cu) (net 2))
 (segment (start 58.61 51.58) (end 59.935 51.58) (width 0.25) (layer F.Cu) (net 2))
 (segment (start 59.935 51.58) (end 59.94 51.575) (width 0.25) (layer F.Cu) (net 2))
 (segment (start 59.415 55.825) (end 59.305 55.825) (width 0.25) (layer F.Cu) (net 2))
 (segment (start 59.305 55.825) (end 58.34 54.86) (width 0.25) (layer F.Cu) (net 2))
 (segment (start 58.34 54.86) (end 58.34 53.875) (width 0.25) (layer F.Cu) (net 2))
 (segment (start 58.34 52.775) (end 58.61 52.505) (width 0.25) (layer F.Cu) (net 2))
 (segment (start 58.61 51.58) (end 58.61 52.505) (width 0.25) (layer F.Cu) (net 2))
 (segment (start 58.34 53.875) (end 58.34 52.775) (width 0.25) (layer F.Cu) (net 2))
 (segment (start 57.34 49.375) (end 58.61 49.375) (width 0.25) (layer F.Cu) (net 2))
 (segment (start 58.6 49.41) (end 58.61 49.41) (width 0.25) (layer F.Cu) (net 2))
 (segment (start 58.6 49.385) (end 58.6 49.41) (width 0.25) (layer F.Cu) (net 2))
 (segment (start 58.61 49.375) (end 58.6 49.385) (width 0.25) (layer F.Cu) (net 2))
 (segment (start 58.61 48.76) (end 58.61 49.41) (width 0.25) (layer F.Cu) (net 2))
 (segment (start 58.61 49.41) (end 58.61 51.58) (width 0.25) (layer F.Cu) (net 2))
 (segment (start 59.64 48.28) (end 58.62 48.28) (width 0.25) (layer F.Cu) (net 2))
 (segment (start 58.62 48.28) (end 58.61 48.29) (width 0.25) (layer F.Cu) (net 2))
 (segment (start 59.63 48.29) (end 59.64 48.28) (width 0.25) (layer F.Cu) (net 2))
 (segment (start 58.03 43.05) (end 58.31 43.05) (width 0.25) (layer F.Cu) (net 2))
 (segment (start 56.365 43.05) (end 57.86 43.05) (width 0.25) (layer F.Cu) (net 2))
 (segment (start 55.39 44.025) (end 56.365 43.05) (width 0.25) (layer F.Cu) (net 2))
 (segment (start 57.86 43.05) (end 58.03 43.05) (width 0.25) (layer F.Cu) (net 2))
 (segment (start 58.31 43.05) (end 58.61 43.35) (width 0.25) (layer F.Cu) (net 2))
 (segment (start 58.61 43.35) (end 58.61 48.29) (width 0.25) (layer F.Cu) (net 2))
 (segment (start 58.61 48.29) (end 58.61 48.76) (width 0.25) (layer F.Cu) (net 2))
 (segment (start 65.965 58.71156) (end 65.1141 59.56246) (width 0.25) (layer F.Cu) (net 2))
 (segment (start 57.24 53.875) (end 57.24 53.85) (width 0.25) (layer F.Cu) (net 2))
 (segment (start 59.94 51.575) (end 59.84 51.575) (width 0.25) (layer F.Cu) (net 2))
 (segment (start 59.415 55.825) (end 59.415 58.86336) (width 0.25) (layer F.Cu) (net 2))
 (segment (start 59.415 58.86336) (end 60.1141 59.56246) (width 0.25) (layer F.Cu) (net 2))
 (segment (start 59.1141 62.26246) (end 66.1141 62.26246) (width 0.25) (layer F.Cu) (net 2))
 (segment (start 59.1141 62.26246) (end 59.1141 60.56246) (width 0.25) (layer F.Cu) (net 2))
 (segment (start 59.1141 60.56246) (end 60.1141 59.56246) (width 0.25) (layer F.Cu) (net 2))
 (segment (start 66.1141 62.26246) (end 66.1141 60.56246) (width 0.25) (layer F.Cu) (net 2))
 (segment (start 66.1141 60.56246) (end 65.1141 59.56246) (width 0.25) (layer F.Cu) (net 2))
 (segment (start 65.1141 59.56246) (end 63.9141 59.56246) (width 0.25) (layer F.Cu) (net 2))
 (segment (start 55.39 44.05) (end 55.39 44.025) (width 0.25) (layer F.Cu) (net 2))
 (segment (start 57.24 53.875) (end 57.465 53.875) (width 0.25) (layer F.Cu) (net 2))
 (via (at 55.39 44.05) (size 0.6) (drill 0.4) (layers F.Cu B.Cu) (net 2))
 (segment (start 52.255 40.225) (end 50.965 38.935) (width 0.25) (layer B.Cu) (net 2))
 (segment (start 55.39 44.05) (end 54.765 43.425) (width 0.25) (layer B.Cu) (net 2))
 (segment (start 54.765 43.425) (end 54.765 40.75) (width 0.25) (layer B.Cu) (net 2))
 (segment (start 54.24 40.225) (end 52.255 40.225) (width 0.25) (layer B.Cu) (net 2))
 (segment (start 54.765 40.75) (end 54.24 40.225) (width 0.25) (layer B.Cu) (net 2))
 (segment (start 65.965 55.825) (end 65.965 58.71156) (width 0.25) (layer F.Cu) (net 2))
 (via (at 53.265 44.05) (size 0.6) (drill 0.4) (layers F.Cu B.Cu) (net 9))
 (segment (start 53.265 44.05) (end 54.8725 45.6575) (width 0.25) (layer B.Cu) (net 9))
 (segment (start 54.265 47.025) (end 54.265 46.265) (width 0.25) (layer B.Cu) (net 9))
 (segment (start 54.265 46.265) (end 54.8725 45.6575) (width 0.25) (layer B.Cu) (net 9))
 (segment (start 64.915 41.7) (end 64.915 42.6) (width 0.25) (layer B.Cu) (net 9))
 (segment (start 64.915 42.6) (end 62.74 44.775) (width 0.25) (layer B.Cu) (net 9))
 (segment (start 62.89 40.2) (end 64.4 40.2) (width 0.25) (layer B.Cu) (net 9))
 (segment (start 64.4 40.2) (end 64.915 40.715) (width 0.25) (layer B.Cu) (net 9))
 (segment (start 62.39 40.2) (end 61.125 38.935) (width 0.25) (layer B.Cu) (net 9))
 (segment (start 55.93898 51.65) (end 55.915 51.65) (width 0.25) (layer F.Cu) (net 9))
 (segment (start 55.915 51.65) (end 54.265 50) (width 0.25) (layer F.Cu) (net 9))
 (segment (start 54.265 50) (end 54.265 47.025) (width 0.25) (layer F.Cu) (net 9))
 (via (at 54.265 47.025) (size 0.6) (drill 0.4) (layers F.Cu B.Cu) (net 9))
 (segment (start 61.115 44.775) (end 62.74 44.775) (width 0.25) (layer B.Cu) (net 9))
 (segment (start 54.8725 45.6575) (end 54.89 45.675) (width 0.25) (layer B.Cu) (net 9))
 (segment (start 54.89 45.675) (end 56.265 45.675) (width 0.25) (layer B.Cu) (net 9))
 (segment (start 57.165 44.775) (end 61.115 44.775) (width 0.25) (layer B.Cu) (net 9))
 (segment (start 56.265 45.675) (end 57.165 44.775) (width 0.25) (layer B.Cu) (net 9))
 (segment (start 62.39 40.2) (end 62.89 40.2) (width 0.25) (layer B.Cu) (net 9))
 (segment (start 64.915 40.715) (end 64.915 41.7) (width 0.25) (layer B.Cu) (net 9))
 (segment (start 59.84098 51.575) (end 57.265 51.575) (width 0.25) (layer B.Cu) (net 3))
 (segment (start 57.265 51.575) (end 53.505 47.815) (width 0.25) (layer B.Cu) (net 3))
 (segment (start 53.505 41.475) (end 53.505 41.66) (width 0.25) (layer B.Cu) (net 3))
 (segment (start 53.505 41.66) (end 51.79 43.375) (width 0.25) (layer B.Cu) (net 3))
 (segment (start 51.79 46.1) (end 53.505 47.815) (width 0.25) (layer B.Cu) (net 3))
 (segment (start 51.79 43.375) (end 51.79 46.1) (width 0.25) (layer B.Cu) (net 3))
 (segment (start 64.715 49.45) (end 66.04 49.45) (width 0.25) (layer B.Cu) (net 1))
 (segment (start 66.042 49.452) (end 66.042 51.562) (width 0.25) (layer F.Cu) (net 1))
 (segment (start 66.04 49.45) (end 66.042 49.452) (width 0.25) (layer F.Cu) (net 1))
 (via (at 66.04 49.45) (size 0.6) (drill 0.4) (layers F.Cu B.Cu) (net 1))
 (segment (start 63.02 48.66) (end 64.03 48.66) (width 0.25) (layer B.Cu) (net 1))
 (segment (start 64.715 49.345) (end 64.715 49.45) (width 0.25) (layer B.Cu) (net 1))
 (segment (start 64.715 49.45) (end 64.715 50.125) (width 0.25) (layer B.Cu) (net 1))
 (segment (start 64.03 48.66) (end 64.715 49.345) (width 0.25) (layer B.Cu) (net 1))
 (segment (start 62.37 48.66) (end 61.99 48.28) (width 0.25) (layer B.Cu) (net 1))
 (segment (start 63.02 48.66) (end 62.37 48.66) (width 0.25) (layer B.Cu) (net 1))
 (segment (start 60.815 47) (end 60.82 47) (width 0.25) (layer B.Cu) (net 1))
 (segment (start 60.82 47) (end 61.6 47.78) (width 0.25) (layer B.Cu) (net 1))
 (segment (start 61.6 47.78) (end 61.99 47.78) (width 0.25) (layer B.Cu) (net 1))
 (segment (start 61.99 48.28) (end 61.99 47.78) (width 0.25) (layer B.Cu) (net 1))
 (segment (start 61.99 47.275) (end 62.265 47) (width 0.25) (layer B.Cu) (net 1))
 (segment (start 61.99 47.78) (end 61.99 47.275) (width 0.25) (layer B.Cu) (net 1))
 (segment (start 55.065 53.26) (end 55.065 52.3) (width 0.25) (layer B.Cu) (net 1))
 (segment (start 64.715 50.125) (end 64.715 54.345) (width 0.25) (layer B.Cu) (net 1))
 (segment (start 55.065 55.775) (end 55.065 53.26) (width 0.25) (layer B.Cu) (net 1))
 (segment (start 55.065 55.775) (end 63.285 55.775) (width 0.25) (layer B.Cu) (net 1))
 (segment (start 63.285 55.775) (end 64.715 54.345) (width 0.25) (layer B.Cu) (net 1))
 (via (at 55.065 55.775) (size 0.6) (drill 0.4) (layers F.Cu B.Cu) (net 1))
 (segment (start 55.065 52.3) (end 52.14 49.375) (width 0.25) (layer B.Cu) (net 1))
 (via (at 52.14 49.375) (size 0.6) (drill 0.4) (layers F.Cu B.Cu) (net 1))
 (segment (start 52.14 49.375) (end 55.065 52.3) (width 0.25) (layer B.Cu) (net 1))
 (segment (start 60.805 47.01) (end 59.64 47.01) (width 0.25) (layer F.Cu) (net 1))
 (segment (start 60.815 47) (end 60.805 47.01) (width 0.25) (layer F.Cu) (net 1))
 (segment (start 50.965 48.2) (end 52.14 49.375) (width 0.25) (layer B.Cu) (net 1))
 (segment (start 50.965 48.125) (end 50.965 48.2) (width 0.25) (layer B.Cu) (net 1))
 (segment (start 50.965 41.475) (end 50.965 48.125) (width 0.25) (layer B.Cu) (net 1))
 (segment (start 65.99 44.47) (end 64.835 44.47) (width 0.25) (layer F.Cu) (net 1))
 (segment (start 64.835 44.47) (end 64.815 44.45) (width 0.25) (layer F.Cu) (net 1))
 (via (at 64.815 44.45) (size 0.6) (drill 0.4) (layers F.Cu B.Cu) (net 1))
 (segment (start 64.815 44.45) (end 62.265 47) (width 0.25) (layer B.Cu) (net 1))
 (segment (start 65.99 44.47) (end 65.99 45.74) (width 0.25) (layer F.Cu) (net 1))
 (via (at 60.815 47) (size 0.6) (drill 0.4) (layers F.Cu B.Cu) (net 1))
 (segment (start 53.505 38.935) (end 53.765 38.935) (width 0.25) (layer B.Cu) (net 4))
 (segment (start 53.765 38.935) (end 55.04 40.21) (width 0.25) (layer B.Cu) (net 4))
 (segment (start 61.725 40.21) (end 62.39 40.875) (width 0.25) (layer B.Cu) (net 4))
 (segment (start 55.04 40.21) (end 61.725 40.21) (width 0.25) (layer B.Cu) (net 4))
 (segment (start 63.35 46.13) (end 64.23 47.01) (width 0.25) (layer F.Cu) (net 4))
 (segment (start 63.35 44.22) (end 63.35 46.13) (width 0.25) (layer F.Cu) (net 4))
 (segment (start 62.39 43.26) (end 63.35 44.22) (width 0.25) (layer F.Cu) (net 4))
 (segment (start 62.39 42.375) (end 62.39 43.26) (width 0.25) (layer F.Cu) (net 4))
 (segment (start 64.23 47.01) (end 65.99 47.01) (width 0.25) (layer F.Cu) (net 4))
 (via (at 62.39 42.375) (size 0.6) (drill 0.4) (layers F.Cu B.Cu) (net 4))
 (segment (start 62.39 40.875) (end 62.39 42.375) (width 0.25) (layer B.Cu) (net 4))
 (segment (start 53.7 38.935) (end 53.505 38.935) (width 0.25) (layer B.Cu) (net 4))
 (segment (start 56.045 38.935) (end 56.265 38.935) (width 0.25) (layer F.Cu) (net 6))
 (segment (start 56.265 38.935) (end 57.53 40.2) (width 0.25) (layer F.Cu) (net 6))
 (segment (start 59.19 40.2) (end 59.865 40.875) (width 0.25) (layer F.Cu) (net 6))
 (segment (start 57.53 40.2) (end 59.19 40.2) (width 0.25) (layer F.Cu) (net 6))
 (segment (start 62.615 44.375) (end 61.365 43.125) (width 0.25) (layer F.Cu) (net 6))
 (segment (start 62.615 45.75) (end 62.615 44.375) (width 0.25) (layer F.Cu) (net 6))
 (segment (start 61.365 43.125) (end 60.79 43.125) (width 0.25) (layer F.Cu) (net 6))
 (segment (start 59.64 45.74) (end 60.75 45.74) (width 0.25) (layer F.Cu) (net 6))
 (segment (start 60.79 45.75) (end 62.615 45.75) (width 0.25) (layer B.Cu) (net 6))
 (segment (start 60.765 45.725) (end 60.79 45.75) (width 0.25) (layer B.Cu) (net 6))
 (via (at 60.765 45.725) (size 0.6) (drill 0.4) (layers F.Cu B.Cu) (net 6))
 (segment (start 60.75 45.74) (end 60.765 45.725) (width 0.25) (layer F.Cu) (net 6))
 (segment (start 59.865 41.525) (end 59.865 42.2) (width 0.25) (layer F.Cu) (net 6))
 (segment (start 59.865 42.2) (end 60.79 43.125) (width 0.25) (layer F.Cu) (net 6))
 (segment (start 61.015 45.75) (end 62.615 45.75) (width 0.25) (layer B.Cu) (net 6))
 (via (at 62.615 45.75) (size 0.6) (drill 0.4) (layers F.Cu B.Cu) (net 6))
 (segment (start 59.865 40.875) (end 59.865 41.525) (width 0.25) (layer F.Cu) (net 6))
 (segment (start 56.045 38.935) (end 56.05 38.935) (width 0.25) (layer F.Cu) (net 6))
 (segment (start 64.57 48.28) (end 65.99 48.28) (width 0.25) (layer F.Cu) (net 8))
 (segment (start 64.565 48.275) (end 64.57 48.28) (width 0.25) (layer F.Cu) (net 8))
 (via (at 64.565 48.275) (size 0.6) (drill 0.4) (layers F.Cu B.Cu) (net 8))
 (segment (start 59 38.935) (end 60.265 40.2) (width 0.25) (layer F.Cu) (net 8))
 (segment (start 66.285 48.28) (end 65.99 48.28) (width 0.25) (layer F.Cu) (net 8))
 (segment (start 58.585 38.935) (end 59 38.935) (width 0.25) (layer F.Cu) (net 8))
 (segment (start 58.585 38.935) (end 58.6 38.935) (width 0.25) (layer F.Cu) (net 8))
 (segment (start 60.265 40.2) (end 64.315 40.2) (width 0.25) (layer F.Cu) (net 8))
 (segment (start 64.315 40.2) (end 64.915 40.8) (width 0.25) (layer F.Cu) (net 8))
 (segment (start 64.915 40.8) (end 64.915 43.425) (width 0.25) (layer F.Cu) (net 8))
 (via (at 64.565 46.375) (size 0.6) (drill 0.4) (layers F.Cu B.Cu) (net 8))
 (segment (start 64.565 46.375) (end 64.565 48.275) (width 0.25) (layer B.Cu) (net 8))
 (segment (start 64.4525 46.2625) (end 64.565 46.375) (width 0.25) (layer F.Cu) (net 8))
 (segment (start 64.04 45.85) (end 64.4525 46.2625) (width 0.25) (layer F.Cu) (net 8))
 (segment (start 64.04 44.3) (end 64.04 45.85) (width 0.25) (layer F.Cu) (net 8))
 (segment (start 64.24 44.1) (end 64.04 44.3) (width 0.25) (layer F.Cu) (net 8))
 (segment (start 64.915 43.425) (end 64.24 44.1) (width 0.25) (layer F.Cu) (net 8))
 (segment (start 61.015 44.075) (end 62.515 44.075) (width 0.25) (layer B.Cu) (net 10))
 (segment (start 63.665 42.925) (end 63.665 41.475) (width 0.25) (layer B.Cu) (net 10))
 (segment (start 62.515 44.075) (end 63.665 42.925) (width 0.25) (layer B.Cu) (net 10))
 (segment (start 57.515 44.075) (end 61.015 44.075) (width 0.25) (layer B.Cu) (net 10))
 (segment (start 57.515 44.075) (end 57.515 44.05) (width 0.25) (layer F.Cu) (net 10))
 (via (at 57.515 44.075) (size 0.6) (drill 0.4) (layers F.Cu B.Cu) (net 10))
 (segment (start 62.64 47.975) (end 62.64 47.36) (width 0.25) (layer B.Cu) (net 11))
 (segment (start 65.1 45.4) (end 66.205 44.295) (width 0.25) (layer B.Cu) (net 11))
 (segment (start 64.6 45.4) (end 65.1 45.4) (width 0.25) (layer B.Cu) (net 11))
 (segment (start 62.64 47.36) (end 64.6 45.4) (width 0.25) (layer B.Cu) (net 11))
 (segment (start 59.64 44.47) (end 61.184998 44.47) (width 0.25) (layer F.Cu) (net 11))
 (via (at 63.165 49.45) (size 0.6) (drill 0.4) (layers F.Cu B.Cu) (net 11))
 (segment (start 61.115 49.45) (end 63.165 49.45) (width 0.25) (layer B.Cu) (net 11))
 (via (at 61.115 49.45) (size 0.6) (drill 0.4) (layers F.Cu B.Cu) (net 11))
 (segment (start 61.514998 49.050002) (end 61.115 49.45) (width 0.25) (layer F.Cu) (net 11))
 (segment (start 61.514998 44.8) (end 61.514998 49.050002) (width 0.25) (layer F.Cu) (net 11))
 (segment (start 61.184998 44.47) (end 61.514998 44.8) (width 0.25) (layer F.Cu) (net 11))
 (segment (start 63.863 50.148) (end 63.165 49.45) (width 0.25) (layer F.Cu) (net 11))
 (segment (start 63.165 49.45) (end 62.715 49) (width 0.25) (layer F.Cu) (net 11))
 (segment (start 64.142 51.562) (end 64.142 50.427) (width 0.25) (layer F.Cu) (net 11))
 (segment (start 64.142 50.427) (end 63.863 50.148) (width 0.25) (layer F.Cu) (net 11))
 (segment (start 66.205 41.475) (end 66.205 42.31) (width 0.25) (layer B.Cu) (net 11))
 (segment (start 62.715 49) (end 62.715 48.05) (width 0.25) (layer F.Cu) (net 11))
 (via (at 62.64 47.975) (size 0.6) (drill 0.4) (layers F.Cu B.Cu) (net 11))
 (segment (start 62.715 48.05) (end 62.64 47.975) (width 0.25) (layer F.Cu) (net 11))
 (segment (start 66.205 41.475) (end 66.205 44.295) (width 0.25) (layer B.Cu) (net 11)))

